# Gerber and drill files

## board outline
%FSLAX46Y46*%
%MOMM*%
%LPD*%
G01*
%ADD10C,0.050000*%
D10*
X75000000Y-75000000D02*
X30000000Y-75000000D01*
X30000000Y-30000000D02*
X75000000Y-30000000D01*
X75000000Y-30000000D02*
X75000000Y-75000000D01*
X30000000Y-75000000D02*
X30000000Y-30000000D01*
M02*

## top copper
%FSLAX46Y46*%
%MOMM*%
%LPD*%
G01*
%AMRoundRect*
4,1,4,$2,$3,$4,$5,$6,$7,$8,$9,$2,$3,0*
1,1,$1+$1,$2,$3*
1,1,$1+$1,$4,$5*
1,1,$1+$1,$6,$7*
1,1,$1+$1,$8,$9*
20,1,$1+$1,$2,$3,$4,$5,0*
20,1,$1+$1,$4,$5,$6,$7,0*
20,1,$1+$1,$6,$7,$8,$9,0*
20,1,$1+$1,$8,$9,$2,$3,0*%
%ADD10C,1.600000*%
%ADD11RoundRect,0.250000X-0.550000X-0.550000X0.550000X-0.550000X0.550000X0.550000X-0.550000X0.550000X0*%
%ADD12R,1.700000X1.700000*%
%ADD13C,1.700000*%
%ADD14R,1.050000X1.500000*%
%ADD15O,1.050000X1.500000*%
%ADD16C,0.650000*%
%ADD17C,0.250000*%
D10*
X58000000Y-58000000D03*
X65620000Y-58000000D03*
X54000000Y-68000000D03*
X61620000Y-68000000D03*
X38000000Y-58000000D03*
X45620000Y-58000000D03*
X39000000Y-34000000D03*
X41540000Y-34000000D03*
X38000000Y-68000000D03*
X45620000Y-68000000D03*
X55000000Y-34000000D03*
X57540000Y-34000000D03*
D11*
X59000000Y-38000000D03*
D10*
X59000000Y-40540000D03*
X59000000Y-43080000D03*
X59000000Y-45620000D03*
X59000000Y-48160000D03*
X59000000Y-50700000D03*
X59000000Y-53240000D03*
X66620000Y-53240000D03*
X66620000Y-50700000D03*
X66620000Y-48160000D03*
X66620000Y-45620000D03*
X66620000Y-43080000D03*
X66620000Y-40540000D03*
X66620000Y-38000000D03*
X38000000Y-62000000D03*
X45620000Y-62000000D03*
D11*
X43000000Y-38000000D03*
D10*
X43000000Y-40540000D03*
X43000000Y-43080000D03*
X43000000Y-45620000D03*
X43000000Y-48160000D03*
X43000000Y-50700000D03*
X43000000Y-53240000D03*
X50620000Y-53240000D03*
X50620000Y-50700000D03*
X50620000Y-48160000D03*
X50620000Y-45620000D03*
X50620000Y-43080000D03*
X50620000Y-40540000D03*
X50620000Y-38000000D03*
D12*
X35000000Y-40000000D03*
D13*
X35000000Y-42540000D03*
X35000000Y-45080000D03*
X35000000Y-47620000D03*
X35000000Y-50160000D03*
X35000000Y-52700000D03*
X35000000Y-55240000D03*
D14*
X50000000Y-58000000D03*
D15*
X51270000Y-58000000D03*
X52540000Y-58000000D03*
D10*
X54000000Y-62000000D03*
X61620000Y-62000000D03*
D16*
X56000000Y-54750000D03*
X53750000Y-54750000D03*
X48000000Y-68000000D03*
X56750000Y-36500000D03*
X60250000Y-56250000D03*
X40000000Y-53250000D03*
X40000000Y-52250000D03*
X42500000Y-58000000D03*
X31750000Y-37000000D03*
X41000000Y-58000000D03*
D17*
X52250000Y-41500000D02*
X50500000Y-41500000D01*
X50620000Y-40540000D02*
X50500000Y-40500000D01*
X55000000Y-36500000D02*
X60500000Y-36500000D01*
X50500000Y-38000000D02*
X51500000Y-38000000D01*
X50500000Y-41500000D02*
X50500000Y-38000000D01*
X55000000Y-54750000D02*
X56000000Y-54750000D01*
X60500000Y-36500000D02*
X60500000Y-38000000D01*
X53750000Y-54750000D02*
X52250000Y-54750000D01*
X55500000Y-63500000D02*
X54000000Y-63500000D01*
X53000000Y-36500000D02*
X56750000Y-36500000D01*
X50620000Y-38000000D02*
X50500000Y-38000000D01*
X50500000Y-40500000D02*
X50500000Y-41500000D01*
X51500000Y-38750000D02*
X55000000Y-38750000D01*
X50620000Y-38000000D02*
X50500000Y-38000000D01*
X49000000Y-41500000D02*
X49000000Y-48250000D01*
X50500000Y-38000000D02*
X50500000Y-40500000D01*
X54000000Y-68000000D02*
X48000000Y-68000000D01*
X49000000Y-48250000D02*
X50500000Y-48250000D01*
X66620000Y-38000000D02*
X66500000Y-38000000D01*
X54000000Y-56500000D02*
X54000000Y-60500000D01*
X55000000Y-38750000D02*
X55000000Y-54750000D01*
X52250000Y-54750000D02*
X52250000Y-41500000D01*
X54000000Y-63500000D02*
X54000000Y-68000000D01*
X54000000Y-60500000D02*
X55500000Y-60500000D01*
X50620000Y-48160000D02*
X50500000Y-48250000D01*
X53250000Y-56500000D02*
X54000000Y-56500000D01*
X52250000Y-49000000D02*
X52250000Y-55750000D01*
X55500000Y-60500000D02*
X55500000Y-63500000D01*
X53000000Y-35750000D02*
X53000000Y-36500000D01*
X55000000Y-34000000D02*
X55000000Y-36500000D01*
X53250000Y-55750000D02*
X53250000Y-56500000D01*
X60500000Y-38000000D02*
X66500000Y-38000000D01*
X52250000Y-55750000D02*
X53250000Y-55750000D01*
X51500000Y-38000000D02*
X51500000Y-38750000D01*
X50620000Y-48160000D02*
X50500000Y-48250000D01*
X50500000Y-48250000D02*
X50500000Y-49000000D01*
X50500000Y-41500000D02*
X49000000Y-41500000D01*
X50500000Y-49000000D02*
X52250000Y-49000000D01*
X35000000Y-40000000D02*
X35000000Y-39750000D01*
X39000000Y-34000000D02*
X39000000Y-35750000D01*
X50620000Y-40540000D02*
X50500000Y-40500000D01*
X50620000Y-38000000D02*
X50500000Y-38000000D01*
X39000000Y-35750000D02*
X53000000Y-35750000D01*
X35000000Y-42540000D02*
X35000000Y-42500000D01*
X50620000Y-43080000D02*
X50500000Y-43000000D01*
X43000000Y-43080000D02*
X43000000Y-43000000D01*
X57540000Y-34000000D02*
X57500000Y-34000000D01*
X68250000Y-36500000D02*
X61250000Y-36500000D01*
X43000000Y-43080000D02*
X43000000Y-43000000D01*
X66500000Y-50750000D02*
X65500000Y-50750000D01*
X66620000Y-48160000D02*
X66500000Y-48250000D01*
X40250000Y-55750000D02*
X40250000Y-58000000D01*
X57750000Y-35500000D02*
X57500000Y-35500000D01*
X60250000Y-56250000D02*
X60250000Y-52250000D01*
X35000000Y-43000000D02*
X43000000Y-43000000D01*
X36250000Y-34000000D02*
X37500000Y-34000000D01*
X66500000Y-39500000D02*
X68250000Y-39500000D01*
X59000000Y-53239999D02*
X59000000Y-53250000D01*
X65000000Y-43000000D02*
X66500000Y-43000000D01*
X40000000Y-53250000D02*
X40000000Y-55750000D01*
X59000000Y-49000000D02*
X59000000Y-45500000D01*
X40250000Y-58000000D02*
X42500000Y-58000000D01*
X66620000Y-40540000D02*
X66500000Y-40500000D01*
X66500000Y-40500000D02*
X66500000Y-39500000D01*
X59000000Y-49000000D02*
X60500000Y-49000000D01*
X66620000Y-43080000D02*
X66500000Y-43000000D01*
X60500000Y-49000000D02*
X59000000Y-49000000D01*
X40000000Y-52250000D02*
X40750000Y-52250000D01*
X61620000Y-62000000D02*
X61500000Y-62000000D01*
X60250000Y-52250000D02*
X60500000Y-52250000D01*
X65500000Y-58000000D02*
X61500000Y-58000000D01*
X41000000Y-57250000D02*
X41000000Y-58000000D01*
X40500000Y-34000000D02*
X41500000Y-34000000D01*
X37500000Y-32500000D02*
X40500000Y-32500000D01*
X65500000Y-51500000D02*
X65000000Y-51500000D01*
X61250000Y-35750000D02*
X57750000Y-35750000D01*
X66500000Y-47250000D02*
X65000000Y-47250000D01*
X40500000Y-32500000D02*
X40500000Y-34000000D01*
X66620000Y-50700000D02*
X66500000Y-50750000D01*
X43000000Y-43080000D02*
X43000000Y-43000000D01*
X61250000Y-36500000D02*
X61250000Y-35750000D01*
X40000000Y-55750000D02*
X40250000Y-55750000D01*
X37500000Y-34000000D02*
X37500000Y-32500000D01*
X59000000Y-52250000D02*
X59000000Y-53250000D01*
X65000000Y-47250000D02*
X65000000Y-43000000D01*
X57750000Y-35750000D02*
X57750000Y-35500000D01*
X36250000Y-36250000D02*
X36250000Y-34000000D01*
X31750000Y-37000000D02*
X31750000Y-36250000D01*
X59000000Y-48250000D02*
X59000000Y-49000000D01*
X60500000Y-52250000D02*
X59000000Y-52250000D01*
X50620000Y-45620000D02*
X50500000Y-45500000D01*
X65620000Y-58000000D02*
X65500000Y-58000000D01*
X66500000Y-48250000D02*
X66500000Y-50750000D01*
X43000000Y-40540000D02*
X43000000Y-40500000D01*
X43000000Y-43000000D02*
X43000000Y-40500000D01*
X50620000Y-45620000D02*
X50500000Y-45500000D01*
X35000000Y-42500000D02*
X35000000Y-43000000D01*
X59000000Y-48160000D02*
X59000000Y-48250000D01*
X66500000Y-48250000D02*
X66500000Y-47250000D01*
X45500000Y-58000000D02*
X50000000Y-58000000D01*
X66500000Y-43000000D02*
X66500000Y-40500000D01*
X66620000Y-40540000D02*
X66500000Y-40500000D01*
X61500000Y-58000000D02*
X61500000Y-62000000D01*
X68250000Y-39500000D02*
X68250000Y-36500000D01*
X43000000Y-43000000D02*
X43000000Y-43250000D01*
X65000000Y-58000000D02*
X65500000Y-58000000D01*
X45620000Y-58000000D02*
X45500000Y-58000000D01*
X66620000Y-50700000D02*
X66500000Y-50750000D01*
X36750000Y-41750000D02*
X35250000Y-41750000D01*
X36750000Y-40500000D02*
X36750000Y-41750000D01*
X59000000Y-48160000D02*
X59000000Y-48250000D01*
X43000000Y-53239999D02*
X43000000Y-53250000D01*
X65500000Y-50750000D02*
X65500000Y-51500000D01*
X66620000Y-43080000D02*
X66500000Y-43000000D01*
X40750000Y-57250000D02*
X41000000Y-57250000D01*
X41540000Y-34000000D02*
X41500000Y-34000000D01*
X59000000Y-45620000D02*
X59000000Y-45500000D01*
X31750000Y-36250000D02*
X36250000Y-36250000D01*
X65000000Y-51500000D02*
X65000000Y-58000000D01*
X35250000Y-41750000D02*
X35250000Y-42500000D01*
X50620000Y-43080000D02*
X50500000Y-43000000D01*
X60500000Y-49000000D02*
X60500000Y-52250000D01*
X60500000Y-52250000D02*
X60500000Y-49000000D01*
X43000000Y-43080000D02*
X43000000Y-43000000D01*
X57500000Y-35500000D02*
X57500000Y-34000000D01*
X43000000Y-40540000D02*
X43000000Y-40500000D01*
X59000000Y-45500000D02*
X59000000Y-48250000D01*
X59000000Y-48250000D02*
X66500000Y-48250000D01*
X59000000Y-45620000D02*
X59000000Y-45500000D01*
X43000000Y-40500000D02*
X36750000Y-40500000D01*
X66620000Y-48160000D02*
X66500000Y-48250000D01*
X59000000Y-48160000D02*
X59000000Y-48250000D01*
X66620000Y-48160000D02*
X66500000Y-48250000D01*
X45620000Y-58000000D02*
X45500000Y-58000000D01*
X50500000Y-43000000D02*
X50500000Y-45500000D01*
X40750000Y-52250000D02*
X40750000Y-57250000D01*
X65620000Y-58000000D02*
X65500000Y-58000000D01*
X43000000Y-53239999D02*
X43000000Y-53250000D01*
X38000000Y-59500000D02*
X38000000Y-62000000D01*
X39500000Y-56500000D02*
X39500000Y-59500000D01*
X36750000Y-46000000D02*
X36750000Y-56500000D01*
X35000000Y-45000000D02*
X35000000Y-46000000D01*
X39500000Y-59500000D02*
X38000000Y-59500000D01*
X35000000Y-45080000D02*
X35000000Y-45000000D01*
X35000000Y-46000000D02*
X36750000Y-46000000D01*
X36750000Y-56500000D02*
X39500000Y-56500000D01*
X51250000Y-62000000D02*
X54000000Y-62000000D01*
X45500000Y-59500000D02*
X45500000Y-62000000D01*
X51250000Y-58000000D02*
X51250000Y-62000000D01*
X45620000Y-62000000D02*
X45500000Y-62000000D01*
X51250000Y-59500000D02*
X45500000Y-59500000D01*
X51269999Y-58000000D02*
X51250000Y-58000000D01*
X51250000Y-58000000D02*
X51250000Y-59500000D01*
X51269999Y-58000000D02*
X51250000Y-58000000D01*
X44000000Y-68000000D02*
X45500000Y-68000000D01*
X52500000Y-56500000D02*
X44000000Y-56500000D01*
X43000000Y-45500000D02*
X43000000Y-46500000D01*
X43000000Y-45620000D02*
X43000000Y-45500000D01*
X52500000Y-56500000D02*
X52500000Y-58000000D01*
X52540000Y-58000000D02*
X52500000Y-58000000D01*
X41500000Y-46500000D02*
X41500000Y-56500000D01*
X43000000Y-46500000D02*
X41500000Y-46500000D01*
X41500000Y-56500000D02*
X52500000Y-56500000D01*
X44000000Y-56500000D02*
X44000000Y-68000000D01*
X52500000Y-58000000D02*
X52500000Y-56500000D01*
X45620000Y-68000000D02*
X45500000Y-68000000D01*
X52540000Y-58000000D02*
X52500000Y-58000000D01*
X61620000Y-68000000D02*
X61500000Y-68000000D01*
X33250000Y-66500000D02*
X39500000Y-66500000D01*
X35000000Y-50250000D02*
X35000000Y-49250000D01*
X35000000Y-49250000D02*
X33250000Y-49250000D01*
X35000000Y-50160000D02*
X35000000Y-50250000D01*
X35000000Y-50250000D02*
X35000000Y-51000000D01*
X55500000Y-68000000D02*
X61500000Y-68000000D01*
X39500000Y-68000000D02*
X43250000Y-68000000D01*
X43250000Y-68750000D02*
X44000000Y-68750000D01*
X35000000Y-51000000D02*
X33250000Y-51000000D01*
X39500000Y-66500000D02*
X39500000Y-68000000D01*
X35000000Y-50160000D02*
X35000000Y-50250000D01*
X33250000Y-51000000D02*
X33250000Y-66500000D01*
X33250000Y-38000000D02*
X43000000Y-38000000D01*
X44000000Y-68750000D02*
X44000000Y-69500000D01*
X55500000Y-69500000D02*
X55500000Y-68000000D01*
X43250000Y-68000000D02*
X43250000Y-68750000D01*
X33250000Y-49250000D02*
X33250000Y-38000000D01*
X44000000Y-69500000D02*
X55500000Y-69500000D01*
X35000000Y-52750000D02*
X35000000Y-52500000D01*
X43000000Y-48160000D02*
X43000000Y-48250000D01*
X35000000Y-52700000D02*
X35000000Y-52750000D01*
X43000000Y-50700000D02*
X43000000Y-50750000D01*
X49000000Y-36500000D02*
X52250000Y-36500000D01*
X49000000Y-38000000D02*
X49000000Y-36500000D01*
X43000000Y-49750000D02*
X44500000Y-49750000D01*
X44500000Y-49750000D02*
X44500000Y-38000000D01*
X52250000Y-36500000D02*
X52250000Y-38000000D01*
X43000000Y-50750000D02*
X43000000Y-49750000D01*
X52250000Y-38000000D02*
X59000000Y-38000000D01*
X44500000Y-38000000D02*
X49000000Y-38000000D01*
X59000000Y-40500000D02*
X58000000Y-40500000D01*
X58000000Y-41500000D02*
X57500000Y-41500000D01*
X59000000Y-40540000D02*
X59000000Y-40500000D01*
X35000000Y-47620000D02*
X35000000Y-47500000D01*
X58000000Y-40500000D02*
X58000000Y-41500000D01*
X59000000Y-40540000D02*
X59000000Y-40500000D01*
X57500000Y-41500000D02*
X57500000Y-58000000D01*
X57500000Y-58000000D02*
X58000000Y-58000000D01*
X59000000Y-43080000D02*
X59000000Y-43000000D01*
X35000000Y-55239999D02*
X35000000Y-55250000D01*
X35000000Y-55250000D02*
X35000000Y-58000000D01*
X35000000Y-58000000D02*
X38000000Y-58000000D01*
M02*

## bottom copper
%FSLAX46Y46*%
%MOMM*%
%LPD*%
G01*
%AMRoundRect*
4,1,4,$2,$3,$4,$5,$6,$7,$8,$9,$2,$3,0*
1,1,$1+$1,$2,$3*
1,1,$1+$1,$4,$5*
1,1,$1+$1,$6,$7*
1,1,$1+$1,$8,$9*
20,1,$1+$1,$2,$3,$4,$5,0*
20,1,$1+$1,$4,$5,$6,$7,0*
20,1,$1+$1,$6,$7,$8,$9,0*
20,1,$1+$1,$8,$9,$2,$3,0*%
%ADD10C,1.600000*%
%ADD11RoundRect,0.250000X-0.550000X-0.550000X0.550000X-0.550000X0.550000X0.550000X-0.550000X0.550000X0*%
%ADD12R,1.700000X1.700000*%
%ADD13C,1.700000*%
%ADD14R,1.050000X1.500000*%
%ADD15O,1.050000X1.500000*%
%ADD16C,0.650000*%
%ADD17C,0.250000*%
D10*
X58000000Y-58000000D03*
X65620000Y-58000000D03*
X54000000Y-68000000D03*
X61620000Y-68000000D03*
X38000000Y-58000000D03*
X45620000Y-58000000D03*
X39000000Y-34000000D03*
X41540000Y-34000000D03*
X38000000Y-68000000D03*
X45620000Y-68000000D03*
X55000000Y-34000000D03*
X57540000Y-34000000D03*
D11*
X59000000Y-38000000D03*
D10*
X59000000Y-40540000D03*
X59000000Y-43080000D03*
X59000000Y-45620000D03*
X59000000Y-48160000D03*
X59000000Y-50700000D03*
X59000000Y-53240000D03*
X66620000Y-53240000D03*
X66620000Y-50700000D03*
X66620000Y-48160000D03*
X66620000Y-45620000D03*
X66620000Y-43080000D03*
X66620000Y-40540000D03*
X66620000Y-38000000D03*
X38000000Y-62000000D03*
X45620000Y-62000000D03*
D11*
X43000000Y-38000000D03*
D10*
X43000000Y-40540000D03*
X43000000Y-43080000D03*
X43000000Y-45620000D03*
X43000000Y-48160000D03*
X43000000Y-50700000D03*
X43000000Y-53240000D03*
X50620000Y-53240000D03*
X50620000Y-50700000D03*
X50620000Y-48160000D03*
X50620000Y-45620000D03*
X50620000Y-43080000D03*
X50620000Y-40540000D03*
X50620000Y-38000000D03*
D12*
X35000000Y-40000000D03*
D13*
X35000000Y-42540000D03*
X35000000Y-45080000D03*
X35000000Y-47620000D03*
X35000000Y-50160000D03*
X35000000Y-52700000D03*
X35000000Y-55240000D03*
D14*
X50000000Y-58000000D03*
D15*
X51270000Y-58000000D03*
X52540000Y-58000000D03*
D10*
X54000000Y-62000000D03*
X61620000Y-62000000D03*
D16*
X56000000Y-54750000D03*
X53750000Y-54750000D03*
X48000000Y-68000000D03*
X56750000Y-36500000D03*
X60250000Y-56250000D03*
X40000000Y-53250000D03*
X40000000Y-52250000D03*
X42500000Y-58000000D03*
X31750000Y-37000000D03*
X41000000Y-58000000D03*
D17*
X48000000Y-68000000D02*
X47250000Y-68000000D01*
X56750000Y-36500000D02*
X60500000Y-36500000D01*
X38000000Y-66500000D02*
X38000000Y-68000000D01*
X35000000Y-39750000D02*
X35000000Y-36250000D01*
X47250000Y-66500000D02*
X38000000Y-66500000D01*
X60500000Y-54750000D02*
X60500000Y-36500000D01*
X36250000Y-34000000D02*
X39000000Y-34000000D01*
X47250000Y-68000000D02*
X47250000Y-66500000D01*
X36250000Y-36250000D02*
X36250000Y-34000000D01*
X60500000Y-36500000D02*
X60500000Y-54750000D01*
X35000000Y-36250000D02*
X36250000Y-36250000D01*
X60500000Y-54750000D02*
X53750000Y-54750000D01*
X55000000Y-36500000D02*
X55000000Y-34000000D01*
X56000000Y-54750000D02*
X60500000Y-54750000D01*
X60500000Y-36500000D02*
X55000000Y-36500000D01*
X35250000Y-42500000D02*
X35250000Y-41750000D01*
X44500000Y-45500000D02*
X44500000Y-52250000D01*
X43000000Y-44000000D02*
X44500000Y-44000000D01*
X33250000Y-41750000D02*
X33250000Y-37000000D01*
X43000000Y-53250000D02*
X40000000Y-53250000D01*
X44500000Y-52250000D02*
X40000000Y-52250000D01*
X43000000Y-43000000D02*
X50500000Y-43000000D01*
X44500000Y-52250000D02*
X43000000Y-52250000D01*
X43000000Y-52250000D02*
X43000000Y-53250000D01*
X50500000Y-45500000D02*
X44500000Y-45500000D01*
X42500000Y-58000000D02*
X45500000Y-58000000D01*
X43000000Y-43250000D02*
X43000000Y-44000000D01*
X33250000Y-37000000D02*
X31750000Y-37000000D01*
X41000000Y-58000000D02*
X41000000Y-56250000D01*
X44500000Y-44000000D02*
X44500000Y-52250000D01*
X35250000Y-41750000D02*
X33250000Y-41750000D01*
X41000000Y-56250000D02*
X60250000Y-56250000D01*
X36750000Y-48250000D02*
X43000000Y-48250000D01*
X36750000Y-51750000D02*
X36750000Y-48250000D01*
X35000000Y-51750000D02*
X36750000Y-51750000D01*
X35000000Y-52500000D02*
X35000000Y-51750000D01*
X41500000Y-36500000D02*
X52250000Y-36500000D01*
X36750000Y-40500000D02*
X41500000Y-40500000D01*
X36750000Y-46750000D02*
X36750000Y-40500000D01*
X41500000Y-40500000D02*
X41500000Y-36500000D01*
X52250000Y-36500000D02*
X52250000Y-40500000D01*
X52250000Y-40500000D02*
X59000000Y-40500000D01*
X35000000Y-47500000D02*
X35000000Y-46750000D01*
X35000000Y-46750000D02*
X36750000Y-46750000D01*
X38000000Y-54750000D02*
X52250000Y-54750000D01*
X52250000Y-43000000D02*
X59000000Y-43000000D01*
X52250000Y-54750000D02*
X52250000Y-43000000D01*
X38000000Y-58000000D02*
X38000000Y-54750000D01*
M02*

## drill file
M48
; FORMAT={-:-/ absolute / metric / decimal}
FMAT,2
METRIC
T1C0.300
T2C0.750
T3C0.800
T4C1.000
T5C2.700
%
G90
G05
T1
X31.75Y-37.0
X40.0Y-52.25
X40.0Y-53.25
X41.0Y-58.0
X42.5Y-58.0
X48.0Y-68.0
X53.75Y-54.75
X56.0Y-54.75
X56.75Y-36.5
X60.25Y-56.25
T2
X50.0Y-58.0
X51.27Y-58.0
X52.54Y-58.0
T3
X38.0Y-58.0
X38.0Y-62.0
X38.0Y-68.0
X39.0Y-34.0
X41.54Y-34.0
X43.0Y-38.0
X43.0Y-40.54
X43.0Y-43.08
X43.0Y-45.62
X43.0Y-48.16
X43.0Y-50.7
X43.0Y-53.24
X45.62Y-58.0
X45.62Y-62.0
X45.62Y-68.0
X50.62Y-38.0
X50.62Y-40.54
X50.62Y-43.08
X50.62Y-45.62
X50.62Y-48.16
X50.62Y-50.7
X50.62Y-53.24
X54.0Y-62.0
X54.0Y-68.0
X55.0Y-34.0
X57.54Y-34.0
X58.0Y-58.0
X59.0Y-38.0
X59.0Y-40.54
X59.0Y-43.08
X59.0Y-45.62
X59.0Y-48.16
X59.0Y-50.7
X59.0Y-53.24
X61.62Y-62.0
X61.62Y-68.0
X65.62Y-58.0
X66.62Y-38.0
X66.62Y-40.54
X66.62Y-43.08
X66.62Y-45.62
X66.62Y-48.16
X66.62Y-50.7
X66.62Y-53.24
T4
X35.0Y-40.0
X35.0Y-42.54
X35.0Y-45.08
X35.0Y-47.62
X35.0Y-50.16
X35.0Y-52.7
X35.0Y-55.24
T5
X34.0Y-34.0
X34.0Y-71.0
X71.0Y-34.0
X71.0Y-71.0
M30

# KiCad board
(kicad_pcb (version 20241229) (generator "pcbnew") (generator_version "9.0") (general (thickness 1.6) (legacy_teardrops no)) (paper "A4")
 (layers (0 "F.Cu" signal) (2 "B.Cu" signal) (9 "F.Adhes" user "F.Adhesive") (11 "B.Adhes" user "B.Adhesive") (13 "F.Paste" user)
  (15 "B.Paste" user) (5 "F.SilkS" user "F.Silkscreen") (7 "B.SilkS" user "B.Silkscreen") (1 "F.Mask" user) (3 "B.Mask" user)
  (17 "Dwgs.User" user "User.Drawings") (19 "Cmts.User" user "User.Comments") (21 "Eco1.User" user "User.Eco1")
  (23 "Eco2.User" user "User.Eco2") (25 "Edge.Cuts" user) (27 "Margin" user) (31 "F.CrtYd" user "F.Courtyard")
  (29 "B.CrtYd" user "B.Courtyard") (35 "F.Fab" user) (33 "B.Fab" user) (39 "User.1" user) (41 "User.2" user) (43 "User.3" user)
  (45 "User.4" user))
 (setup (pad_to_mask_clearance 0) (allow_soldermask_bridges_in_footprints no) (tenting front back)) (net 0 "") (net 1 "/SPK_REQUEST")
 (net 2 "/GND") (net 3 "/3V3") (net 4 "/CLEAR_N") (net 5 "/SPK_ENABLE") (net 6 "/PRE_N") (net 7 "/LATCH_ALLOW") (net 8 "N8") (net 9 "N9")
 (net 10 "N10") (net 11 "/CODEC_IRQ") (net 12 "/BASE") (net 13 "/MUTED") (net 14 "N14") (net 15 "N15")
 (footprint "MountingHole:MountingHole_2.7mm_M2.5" (layer "F.Cu") (at 34 71)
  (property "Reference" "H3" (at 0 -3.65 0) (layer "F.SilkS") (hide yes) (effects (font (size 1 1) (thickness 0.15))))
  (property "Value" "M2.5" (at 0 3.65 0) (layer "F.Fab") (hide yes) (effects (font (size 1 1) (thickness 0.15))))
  (pad "" np_thru_hole circle (at 0 0) (size 2.7 2.7) (drill 2.7) (layers "*.Cu" "*.Mask")))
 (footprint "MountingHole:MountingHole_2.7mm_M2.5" (layer "F.Cu") (at 71 71)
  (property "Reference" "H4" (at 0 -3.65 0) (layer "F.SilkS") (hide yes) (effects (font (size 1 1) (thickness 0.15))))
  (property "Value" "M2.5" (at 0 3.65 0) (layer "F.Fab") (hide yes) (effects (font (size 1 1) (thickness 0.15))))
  (pad "" np_thru_hole circle (at 0 0) (size 2.7 2.7) (drill 2.7) (layers "*.Cu" "*.Mask")))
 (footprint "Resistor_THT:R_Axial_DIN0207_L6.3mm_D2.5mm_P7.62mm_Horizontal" (layer "F.Cu") (at 58 58)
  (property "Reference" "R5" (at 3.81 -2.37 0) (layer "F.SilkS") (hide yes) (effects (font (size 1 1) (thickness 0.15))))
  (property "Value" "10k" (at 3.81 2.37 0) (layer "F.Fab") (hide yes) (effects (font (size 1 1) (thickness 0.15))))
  (pad "1" thru_hole circle (at 0 0) (size 1.6 1.6) (drill 0.8) (layers "*.Cu" "*.Mask") (remove_unused_layers no) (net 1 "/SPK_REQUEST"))
  (pad "2" thru_hole circle (at 7.62 0) (size 1.6 1.6) (drill 0.8) (layers "*.Cu" "*.Mask") (remove_unused_layers no) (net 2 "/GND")))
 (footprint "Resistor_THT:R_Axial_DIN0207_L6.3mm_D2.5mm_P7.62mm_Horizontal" (layer "F.Cu") (at 54 68)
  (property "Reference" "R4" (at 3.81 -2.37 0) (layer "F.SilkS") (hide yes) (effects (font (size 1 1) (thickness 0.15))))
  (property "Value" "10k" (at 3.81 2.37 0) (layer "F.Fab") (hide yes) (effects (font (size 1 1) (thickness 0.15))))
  (pad "1" thru_hole circle (at 0 0) (size 1.6 1.6) (drill 0.8) (layers "*.Cu" "*.Mask") (remove_unused_layers no) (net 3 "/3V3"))
  (pad "2" thru_hole circle (at 7.62 0) (size 1.6 1.6) (drill 0.8) (layers "*.Cu" "*.Mask") (remove_unused_layers no) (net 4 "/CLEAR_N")))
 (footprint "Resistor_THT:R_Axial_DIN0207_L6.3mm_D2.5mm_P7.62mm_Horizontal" (layer "F.Cu") (at 38 58)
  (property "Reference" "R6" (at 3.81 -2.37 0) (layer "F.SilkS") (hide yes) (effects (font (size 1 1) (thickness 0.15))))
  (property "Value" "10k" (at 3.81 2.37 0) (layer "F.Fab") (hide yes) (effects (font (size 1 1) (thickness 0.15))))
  (pad "1" thru_hole circle (at 0 0) (size 1.6 1.6) (drill 0.8) (layers "*.Cu" "*.Mask") (remove_unused_layers no) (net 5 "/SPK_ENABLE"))
  (pad "2" thru_hole circle (at 7.62 0) (size 1.6 1.6) (drill 0.8) (layers "*.Cu" "*.Mask") (remove_unused_layers no) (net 2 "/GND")))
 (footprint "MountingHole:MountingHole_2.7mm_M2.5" (layer "F.Cu") (at 34 34)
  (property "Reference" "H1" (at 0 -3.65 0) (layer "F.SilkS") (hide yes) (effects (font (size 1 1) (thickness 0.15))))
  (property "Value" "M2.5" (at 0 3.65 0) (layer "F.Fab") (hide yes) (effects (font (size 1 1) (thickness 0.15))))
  (pad "" np_thru_hole circle (at 0 0) (size 2.7 2.7) (drill 2.7) (layers "*.Cu" "*.Mask")))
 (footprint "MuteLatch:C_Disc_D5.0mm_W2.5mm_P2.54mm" (layer "F.Cu") (at 39 34)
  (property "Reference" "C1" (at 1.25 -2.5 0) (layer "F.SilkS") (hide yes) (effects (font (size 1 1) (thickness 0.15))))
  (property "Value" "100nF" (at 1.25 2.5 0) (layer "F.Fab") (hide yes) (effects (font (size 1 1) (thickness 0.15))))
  (pad "1" thru_hole circle (at 0 0) (size 1.6 1.6) (drill 0.8) (layers "*.Cu" "*.Mask") (remove_unused_layers no) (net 3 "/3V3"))
  (pad "2" thru_hole circle (at 2.54 0) (size 1.6 1.6) (drill 0.8) (layers "*.Cu" "*.Mask") (remove_unused_layers no) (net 2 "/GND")))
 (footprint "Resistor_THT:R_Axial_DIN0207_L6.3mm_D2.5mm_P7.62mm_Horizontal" (layer "F.Cu") (at 38 68)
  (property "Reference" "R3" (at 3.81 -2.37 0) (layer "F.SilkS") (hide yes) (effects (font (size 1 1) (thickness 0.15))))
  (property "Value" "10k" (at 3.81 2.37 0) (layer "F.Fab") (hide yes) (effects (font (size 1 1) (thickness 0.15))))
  (pad "1" thru_hole circle (at 0 0) (size 1.6 1.6) (drill 0.8) (layers "*.Cu" "*.Mask") (remove_unused_layers no) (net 3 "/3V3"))
  (pad "2" thru_hole circle (at 7.62 0) (size 1.6 1.6) (drill 0.8) (layers "*.Cu" "*.Mask") (remove_unused_layers no) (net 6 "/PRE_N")))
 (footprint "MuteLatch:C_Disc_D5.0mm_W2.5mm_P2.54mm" (layer "F.Cu") (at 55 34)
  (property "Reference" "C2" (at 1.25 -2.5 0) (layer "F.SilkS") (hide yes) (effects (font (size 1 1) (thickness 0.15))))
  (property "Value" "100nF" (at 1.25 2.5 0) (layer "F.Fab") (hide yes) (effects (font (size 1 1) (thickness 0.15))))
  (pad "1" thru_hole circle (at 0 0) (size 1.6 1.6) (drill 0.8) (layers "*.Cu" "*.Mask") (remove_unused_layers no) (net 3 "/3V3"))
  (pad "2" thru_hole circle (at 2.54 0) (size 1.6 1.6) (drill 0.8) (layers "*.Cu" "*.Mask") (remove_unused_layers no) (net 2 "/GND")))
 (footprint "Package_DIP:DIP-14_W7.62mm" (layer "F.Cu") (at 59 38)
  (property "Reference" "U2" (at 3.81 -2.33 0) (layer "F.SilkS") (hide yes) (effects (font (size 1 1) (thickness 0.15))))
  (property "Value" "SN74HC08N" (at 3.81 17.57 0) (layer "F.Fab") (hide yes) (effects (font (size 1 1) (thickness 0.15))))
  (pad "1" thru_hole roundrect (at 0 0) (size 1.6 1.6) (drill 0.8) (layers "*.Cu" "*.Mask") (remove_unused_layers no)
   (roundrect_rratio 0.15625) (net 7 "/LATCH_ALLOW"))
  (pad "2" thru_hole circle (at 0 2.54) (size 1.6 1.6) (drill 0.8) (layers "*.Cu" "*.Mask") (remove_unused_layers no) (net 1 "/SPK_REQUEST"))
  (pad "3" thru_hole circle (at 0 5.08) (size 1.6 1.6) (drill 0.8) (layers "*.Cu" "*.Mask") (remove_unused_layers no) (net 5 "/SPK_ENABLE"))
  (pad "4" thru_hole circle (at 0 7.62) (size 1.6 1.6) (drill 0.8) (layers "*.Cu" "*.Mask") (remove_unused_layers no) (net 2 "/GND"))
  (pad "5" thru_hole circle (at 0 10.16) (size 1.6 1.6) (drill 0.8) (layers "*.Cu" "*.Mask") (remove_unused_layers no) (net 2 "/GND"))
  (pad "6" thru_hole circle (at 0 12.7) (size 1.6 1.6) (drill 0.8) (layers "*.Cu" "*.Mask") (remove_unused_layers no) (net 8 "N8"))
  (pad "7" thru_hole circle (at 0 15.24) (size 1.6 1.6) (drill 0.8) (layers "*.Cu" "*.Mask") (remove_unused_layers no) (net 2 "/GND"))
  (pad "8" thru_hole circle (at 7.62 15.24) (size 1.6 1.6) (drill 0.8) (layers "*.Cu" "*.Mask") (remove_unused_layers no) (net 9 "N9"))
  (pad "9" thru_hole circle (at 7.62 12.7) (size 1.6 1.6) (drill 0.8) (layers "*.Cu" "*.Mask") (remove_unused_layers no) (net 2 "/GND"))
  (pad "10" thru_hole circle (at 7.62 10.16) (size 1.6 1.6) (drill 0.8) (layers "*.Cu" "*.Mask") (remove_unused_layers no) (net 2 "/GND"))
  (pad "11" thru_hole circle (at 7.62 7.62) (size 1.6 1.6) (drill 0.8) (layers "*.Cu" "*.Mask") (remove_unused_layers no) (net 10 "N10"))
  (pad "12" thru_hole circle (at 7.62 5.08) (size 1.6 1.6) (drill 0.8) (layers "*.Cu" "*.Mask") (remove_unused_layers no) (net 2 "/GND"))
  (pad "13" thru_hole circle (at 7.62 2.54) (size 1.6 1.6) (drill 0.8) (layers "*.Cu" "*.Mask") (remove_unused_layers no) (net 2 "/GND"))
  (pad "14" thru_hole circle (at 7.62 0) (size 1.6 1.6) (drill 0.8) (layers "*.Cu" "*.Mask") (remove_unused_layers no) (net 3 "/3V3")))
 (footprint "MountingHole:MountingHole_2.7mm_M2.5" (layer "F.Cu") (at 71 34)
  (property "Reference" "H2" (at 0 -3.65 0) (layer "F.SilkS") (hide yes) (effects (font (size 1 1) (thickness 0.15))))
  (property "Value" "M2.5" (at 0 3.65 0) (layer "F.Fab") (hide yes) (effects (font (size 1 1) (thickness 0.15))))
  (pad "" np_thru_hole circle (at 0 0) (size 2.7 2.7) (drill 2.7) (layers "*.Cu" "*.Mask")))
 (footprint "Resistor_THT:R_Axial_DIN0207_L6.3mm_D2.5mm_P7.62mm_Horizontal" (layer "F.Cu") (at 38 62)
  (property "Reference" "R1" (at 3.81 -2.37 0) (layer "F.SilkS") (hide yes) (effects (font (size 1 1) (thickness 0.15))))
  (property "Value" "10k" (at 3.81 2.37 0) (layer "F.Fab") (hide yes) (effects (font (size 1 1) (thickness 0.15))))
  (pad "1" thru_hole circle (at 0 0) (size 1.6 1.6) (drill 0.8) (layers "*.Cu" "*.Mask") (remove_unused_layers no) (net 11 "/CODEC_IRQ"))
  (pad "2" thru_hole circle (at 7.62 0) (size 1.6 1.6) (drill 0.8) (layers "*.Cu" "*.Mask") (remove_unused_layers no) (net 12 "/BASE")))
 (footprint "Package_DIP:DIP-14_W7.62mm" (layer "F.Cu") (at 43 38)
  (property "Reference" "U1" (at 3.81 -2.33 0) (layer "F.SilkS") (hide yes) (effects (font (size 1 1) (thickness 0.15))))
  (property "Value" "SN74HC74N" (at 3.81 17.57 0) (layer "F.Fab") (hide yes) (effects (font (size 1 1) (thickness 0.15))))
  (pad "1" thru_hole roundrect (at 0 0) (size 1.6 1.6) (drill 0.8) (layers "*.Cu" "*.Mask") (remove_unused_layers no)
   (roundrect_rratio 0.15625) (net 4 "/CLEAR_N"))
  (pad "2" thru_hole circle (at 0 2.54) (size 1.6 1.6) (drill 0.8) (layers "*.Cu" "*.Mask") (remove_unused_layers no) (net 2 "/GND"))
  (pad "3" thru_hole circle (at 0 5.08) (size 1.6 1.6) (drill 0.8) (layers "*.Cu" "*.Mask") (remove_unused_layers no) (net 2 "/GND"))
  (pad "4" thru_hole circle (at 0 7.62) (size 1.6 1.6) (drill 0.8) (layers "*.Cu" "*.Mask") (remove_unused_layers no) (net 6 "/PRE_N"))
  (pad "5" thru_hole circle (at 0 10.16) (size 1.6 1.6) (drill 0.8) (layers "*.Cu" "*.Mask") (remove_unused_layers no) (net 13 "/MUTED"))
  (pad "6" thru_hole circle (at 0 12.7) (size 1.6 1.6) (drill 0.8) (layers "*.Cu" "*.Mask") (remove_unused_layers no) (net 7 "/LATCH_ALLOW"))
  (pad "7" thru_hole circle (at 0 15.24) (size 1.6 1.6) (drill 0.8) (layers "*.Cu" "*.Mask") (remove_unused_layers no) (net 2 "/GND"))
  (pad "8" thru_hole circle (at 7.62 15.24) (size 1.6 1.6) (drill 0.8) (layers "*.Cu" "*.Mask") (remove_unused_layers no) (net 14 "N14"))
  (pad "9" thru_hole circle (at 7.62 12.7) (size 1.6 1.6) (drill 0.8) (layers "*.Cu" "*.Mask") (remove_unused_layers no) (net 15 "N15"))
  (pad "10" thru_hole circle (at 7.62 10.16) (size 1.6 1.6) (drill 0.8) (layers "*.Cu" "*.Mask") (remove_unused_layers no) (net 3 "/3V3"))
  (pad "11" thru_hole circle (at 7.62 7.62) (size 1.6 1.6) (drill 0.8) (layers "*.Cu" "*.Mask") (remove_unused_layers no) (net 2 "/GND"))
  (pad "12" thru_hole circle (at 7.62 5.08) (size 1.6 1.6) (drill 0.8) (layers "*.Cu" "*.Mask") (remove_unused_layers no) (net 2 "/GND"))
  (pad "13" thru_hole circle (at 7.62 2.54) (size 1.6 1.6) (drill 0.8) (layers "*.Cu" "*.Mask") (remove_unused_layers no) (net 3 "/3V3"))
  (pad "14" thru_hole circle (at 7.62 0) (size 1.6 1.6) (drill 0.8) (layers "*.Cu" "*.Mask") (remove_unused_layers no) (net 3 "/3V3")))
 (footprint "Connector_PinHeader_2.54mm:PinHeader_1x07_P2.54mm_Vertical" (layer "F.Cu") (at 35 40)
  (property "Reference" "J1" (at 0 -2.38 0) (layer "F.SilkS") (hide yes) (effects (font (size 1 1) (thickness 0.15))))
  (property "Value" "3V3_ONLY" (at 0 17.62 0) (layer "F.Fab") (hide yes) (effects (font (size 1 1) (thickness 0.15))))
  (pad "1" thru_hole rect (at 0 0) (size 1.7 1.7) (drill 1) (layers "*.Cu" "*.Mask") (remove_unused_layers no) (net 3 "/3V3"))
  (pad "2" thru_hole circle (at 0 2.54) (size 1.7 1.7) (drill 1) (layers "*.Cu" "*.Mask") (remove_unused_layers no) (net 2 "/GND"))
  (pad "3" thru_hole circle (at 0 5.08) (size 1.7 1.7) (drill 1) (layers "*.Cu" "*.Mask") (remove_unused_layers no) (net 11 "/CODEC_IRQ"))
  (pad "4" thru_hole circle (at 0 7.62) (size 1.7 1.7) (drill 1) (layers "*.Cu" "*.Mask") (remove_unused_layers no) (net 1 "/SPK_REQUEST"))
  (pad "5" thru_hole circle (at 0 10.16) (size 1.7 1.7) (drill 1) (layers "*.Cu" "*.Mask") (remove_unused_layers no) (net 4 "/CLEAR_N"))
  (pad "6" thru_hole circle (at 0 12.7) (size 1.7 1.7) (drill 1) (layers "*.Cu" "*.Mask") (remove_unused_layers no) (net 13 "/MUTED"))
  (pad "7" thru_hole circle (at 0 15.24) (size 1.7 1.7) (drill 1) (layers "*.Cu" "*.Mask") (remove_unused_layers no) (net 5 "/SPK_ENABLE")))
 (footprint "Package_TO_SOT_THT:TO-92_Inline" (layer "F.Cu") (at 50 58)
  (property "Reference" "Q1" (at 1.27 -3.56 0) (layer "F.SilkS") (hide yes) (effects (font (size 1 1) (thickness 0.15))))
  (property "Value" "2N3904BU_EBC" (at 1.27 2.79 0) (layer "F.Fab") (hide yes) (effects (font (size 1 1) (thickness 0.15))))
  (pad "1" thru_hole rect (at 0 0) (size 1.05 1.5) (drill 0.75) (layers "*.Cu" "*.Mask") (remove_unused_layers no) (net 2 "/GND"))
  (pad "2" thru_hole oval (at 1.27 0) (size 1.05 1.5) (drill 0.75) (layers "*.Cu" "*.Mask") (remove_unused_layers no) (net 12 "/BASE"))
  (pad "3" thru_hole oval (at 2.54 0) (size 1.05 1.5) (drill 0.75) (layers "*.Cu" "*.Mask") (remove_unused_layers no) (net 6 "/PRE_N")))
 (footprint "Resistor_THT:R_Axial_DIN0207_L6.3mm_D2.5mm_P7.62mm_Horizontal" (layer "F.Cu") (at 54 62)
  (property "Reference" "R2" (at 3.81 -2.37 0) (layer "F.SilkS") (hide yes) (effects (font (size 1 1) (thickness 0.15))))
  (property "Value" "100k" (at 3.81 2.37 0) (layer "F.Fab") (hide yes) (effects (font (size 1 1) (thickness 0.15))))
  (pad "1" thru_hole circle (at 0 0) (size 1.6 1.6) (drill 0.8) (layers "*.Cu" "*.Mask") (remove_unused_layers no) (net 12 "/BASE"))
  (pad "2" thru_hole circle (at 7.62 0) (size 1.6 1.6) (drill 0.8) (layers "*.Cu" "*.Mask") (remove_unused_layers no) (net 2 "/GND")))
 (gr_line (start 75 75) (end 30 75) (stroke (width 0.05) (type default)) (layer "Edge.Cuts"))
 (gr_line (start 30 30) (end 75 30) (stroke (width 0.05) (type default)) (layer "Edge.Cuts"))
 (gr_line (start 75 30) (end 75 75) (stroke (width 0.05) (type default)) (layer "Edge.Cuts"))
 (gr_line (start 30 75) (end 30 30) (stroke (width 0.05) (type default)) (layer "Edge.Cuts"))
 (segment (start 52.25 41.5) (end 50.5 41.5) (width 0.25) (layer "F.Cu") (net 3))
 (segment (start 50.62 40.54) (end 50.5 40.5) (width 0.25) (layer "F.Cu") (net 3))
 (segment (start 55 36.5) (end 60.5 36.5) (width 0.25) (layer "F.Cu") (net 3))
 (segment (start 50.5 38) (end 51.5 38) (width 0.25) (layer "F.Cu") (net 3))
 (segment (start 50.5 41.5) (end 50.5 38) (width 0.25) (layer "F.Cu") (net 3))
 (segment (start 55 54.75) (end 56 54.75) (width 0.25) (layer "F.Cu") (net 3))
 (segment (start 60.5 36.5) (end 60.5 38) (width 0.25) (layer "F.Cu") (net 3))
 (segment (start 53.75 54.75) (end 52.25 54.75) (width 0.25) (layer "F.Cu") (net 3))
 (segment (start 55.5 63.5) (end 54 63.5) (width 0.25) (layer "F.Cu") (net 3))
 (segment (start 53 36.5) (end 56.75 36.5) (width 0.25) (layer "F.Cu") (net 3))
 (segment (start 50.62 38) (end 50.5 38) (width 0.25) (layer "F.Cu") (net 3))
 (segment (start 50.5 40.5) (end 50.5 41.5) (width 0.25) (layer "F.Cu") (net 3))
 (segment (start 51.5 38.75) (end 55 38.75) (width 0.25) (layer "F.Cu") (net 3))
 (segment (start 50.62 38) (end 50.5 38) (width 0.25) (layer "F.Cu") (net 3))
 (segment (start 49 41.5) (end 49 48.25) (width 0.25) (layer "F.Cu") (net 3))
 (segment (start 50.5 38) (end 50.5 40.5) (width 0.25) (layer "F.Cu") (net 3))
 (segment (start 54 68) (end 48 68) (width 0.25) (layer "F.Cu") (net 3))
 (segment (start 49 48.25) (end 50.5 48.25) (width 0.25) (layer "F.Cu") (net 3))
 (segment (start 66.62 38) (end 66.5 38) (width 0.25) (layer "F.Cu") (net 3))
 (segment (start 54 56.5) (end 54 60.5) (width 0.25) (layer "F.Cu") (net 3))
 (segment (start 55 38.75) (end 55 54.75) (width 0.25) (layer "F.Cu") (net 3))
 (segment (start 52.25 54.75) (end 52.25 41.5) (width 0.25) (layer "F.Cu") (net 3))
 (segment (start 54 63.5) (end 54 68) (width 0.25) (layer "F.Cu") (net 3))
 (segment (start 54 60.5) (end 55.5 60.5) (width 0.25) (layer "F.Cu") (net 3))
 (segment (start 50.62 48.16) (end 50.5 48.25) (width 0.25) (layer "F.Cu") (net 3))
 (segment (start 53.25 56.5) (end 54 56.5) (width 0.25) (layer "F.Cu") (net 3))
 (segment (start 52.25 49) (end 52.25 55.75) (width 0.25) (layer "F.Cu") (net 3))
 (segment (start 55.5 60.5) (end 55.5 63.5) (width 0.25) (layer "F.Cu") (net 3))
 (segment (start 53 35.75) (end 53 36.5) (width 0.25) (layer "F.Cu") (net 3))
 (segment (start 55 34) (end 55 36.5) (width 0.25) (layer "F.Cu") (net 3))
 (segment (start 53.25 55.75) (end 53.25 56.5) (width 0.25) (layer "F.Cu") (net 3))
 (segment (start 60.5 38) (end 66.5 38) (width 0.25) (layer "F.Cu") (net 3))
 (segment (start 52.25 55.75) (end 53.25 55.75) (width 0.25) (layer "F.Cu") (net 3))
 (segment (start 51.5 38) (end 51.5 38.75) (width 0.25) (layer "F.Cu") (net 3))
 (segment (start 50.62 48.16) (end 50.5 48.25) (width 0.25) (layer "F.Cu") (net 3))
 (segment (start 50.5 48.25) (end 50.5 49) (width 0.25) (layer "F.Cu") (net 3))
 (segment (start 50.5 41.5) (end 49 41.5) (width 0.25) (layer "F.Cu") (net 3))
 (segment (start 50.5 49) (end 52.25 49) (width 0.25) (layer "F.Cu") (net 3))
 (segment (start 35 40) (end 35 39.75) (width 0.25) (layer "F.Cu") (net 3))
 (segment (start 39 34) (end 39 35.75) (width 0.25) (layer "F.Cu") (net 3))
 (segment (start 50.62 40.54) (end 50.5 40.5) (width 0.25) (layer "F.Cu") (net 3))
 (segment (start 50.62 38) (end 50.5 38) (width 0.25) (layer "F.Cu") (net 3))
 (segment (start 39 35.75) (end 53 35.75) (width 0.25) (layer "F.Cu") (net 3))
 (via (at 56 54.75) (size 0.65) (drill 0.3) (layers "F.Cu" "B.Cu") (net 3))
 (via (at 53.75 54.75) (size 0.65) (drill 0.3) (layers "F.Cu" "B.Cu") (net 3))
 (via (at 48 68) (size 0.65) (drill 0.3) (layers "F.Cu" "B.Cu") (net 3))
 (via (at 56.75 36.5) (size 0.65) (drill 0.3) (layers "F.Cu" "B.Cu") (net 3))
 (segment (start 48 68) (end 47.25 68) (width 0.25) (layer "B.Cu") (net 3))
 (segment (start 56.75 36.5) (end 60.5 36.5) (width 0.25) (layer "B.Cu") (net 3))
 (segment (start 38 66.5) (end 38 68) (width 0.25) (layer "B.Cu") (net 3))
 (segment (start 35 39.75) (end 35 36.25) (width 0.25) (layer "B.Cu") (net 3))
 (segment (start 47.25 66.5) (end 38 66.5) (width 0.25) (layer "B.Cu") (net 3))
 (segment (start 60.5 54.75) (end 60.5 36.5) (width 0.25) (layer "B.Cu") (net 3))
 (segment (start 36.25 34) (end 39 34) (width 0.25) (layer "B.Cu") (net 3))
 (segment (start 47.25 68) (end 47.25 66.5) (width 0.25) (layer "B.Cu") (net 3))
 (segment (start 36.25 36.25) (end 36.25 34) (width 0.25) (layer "B.Cu") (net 3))
 (segment (start 60.5 36.5) (end 60.5 54.75) (width 0.25) (layer "B.Cu") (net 3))
 (segment (start 35 36.25) (end 36.25 36.25) (width 0.25) (layer "B.Cu") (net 3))
 (segment (start 60.5 54.75) (end 53.75 54.75) (width 0.25) (layer "B.Cu") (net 3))
 (segment (start 55 36.5) (end 55 34) (width 0.25) (layer "B.Cu") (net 3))
 (segment (start 56 54.75) (end 60.5 54.75) (width 0.25) (layer "B.Cu") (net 3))
 (segment (start 60.5 36.5) (end 55 36.5) (width 0.25) (layer "B.Cu") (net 3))
 (segment (start 35 42.54) (end 35 42.5) (width 0.25) (layer "F.Cu") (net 2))
 (segment (start 50.62 43.08) (end 50.5 43) (width 0.25) (layer "F.Cu") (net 2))
 (segment (start 43 43.08) (end 43 43) (width 0.25) (layer "F.Cu") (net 2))
 (segment (start 57.54 34) (end 57.5 34) (width 0.25) (layer "F.Cu") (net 2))
 (segment (start 68.25 36.5) (end 61.25 36.5) (width 0.25) (layer "F.Cu") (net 2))
 (segment (start 43 43.08) (end 43 43) (width 0.25) (layer "F.Cu") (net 2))
 (segment (start 66.5 50.75) (end 65.5 50.75) (width 0.25) (layer "F.Cu") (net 2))
 (segment (start 66.62 48.16) (end 66.5 48.25) (width 0.25) (layer "F.Cu") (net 2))
 (segment (start 40.25 55.75) (end 40.25 58) (width 0.25) (layer "F.Cu") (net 2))
 (segment (start 57.75 35.5) (end 57.5 35.5) (width 0.25) (layer "F.Cu") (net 2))
 (segment (start 60.25 56.25) (end 60.25 52.25) (width 0.25) (layer "F.Cu") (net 2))
 (segment (start 35 43) (end 43 43) (width 0.25) (layer "F.Cu") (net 2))
 (segment (start 36.25 34) (end 37.5 34) (width 0.25) (layer "F.Cu") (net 2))
 (segment (start 66.5 39.5) (end 68.25 39.5) (width 0.25) (layer "F.Cu") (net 2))
 (segment (start 59 53.239999) (end 59 53.25) (width 0.25) (layer "F.Cu") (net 2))
 (segment (start 65 43) (end 66.5 43) (width 0.25) (layer "F.Cu") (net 2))
 (segment (start 40 53.25) (end 40 55.75) (width 0.25) (layer "F.Cu") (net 2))
 (segment (start 59 49) (end 59 45.5) (width 0.25) (layer "F.Cu") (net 2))
 (segment (start 40.25 58) (end 42.5 58) (width 0.25) (layer "F.Cu") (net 2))
 (segment (start 66.62 40.54) (end 66.5 40.5) (width 0.25) (layer "F.Cu") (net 2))
 (segment (start 66.5 40.5) (end 66.5 39.5) (width 0.25) (layer "F.Cu") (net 2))
 (segment (start 59 49) (end 60.5 49) (width 0.25) (layer "F.Cu") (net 2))
 (segment (start 66.62 43.08) (end 66.5 43) (width 0.25) (layer "F.Cu") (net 2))
 (segment (start 60.5 49) (end 59 49) (width 0.25) (layer "F.Cu") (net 2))
 (segment (start 40 52.25) (end 40.75 52.25) (width 0.25) (layer "F.Cu") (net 2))
 (segment (start 61.62 62) (end 61.5 62) (width 0.25) (layer "F.Cu") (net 2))
 (segment (start 60.25 52.25) (end 60.5 52.25) (width 0.25) (layer "F.Cu") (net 2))
 (segment (start 65.5 58) (end 61.5 58) (width 0.25) (layer "F.Cu") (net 2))
 (segment (start 41 57.25) (end 41 58) (width 0.25) (layer "F.Cu") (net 2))
 (segment (start 40.5 34) (end 41.5 34) (width 0.25) (layer "F.Cu") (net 2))
 (segment (start 37.5 32.5) (end 40.5 32.5) (width 0.25) (layer "F.Cu") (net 2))
 (segment (start 65.5 51.5) (end 65 51.5) (width 0.25) (layer "F.Cu") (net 2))
 (segment (start 61.25 35.75) (end 57.75 35.75) (width 0.25) (layer "F.Cu") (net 2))
 (segment (start 66.5 47.25) (end 65 47.25) (width 0.25) (layer "F.Cu") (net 2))
 (segment (start 40.5 32.5) (end 40.5 34) (width 0.25) (layer "F.Cu") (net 2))
 (segment (start 66.62 50.7) (end 66.5 50.75) (width 0.25) (layer "F.Cu") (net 2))
 (segment (start 43 43.08) (end 43 43) (width 0.25) (layer "F.Cu") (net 2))
 (segment (start 61.25 36.5) (end 61.25 35.75) (width 0.25) (layer "F.Cu") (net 2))
 (segment (start 40 55.75) (end 40.25 55.75) (width 0.25) (layer "F.Cu") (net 2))
 (segment (start 37.5 34) (end 37.5 32.5) (width 0.25) (layer "F.Cu") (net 2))
 (segment (start 59 52.25) (end 59 53.25) (width 0.25) (layer "F.Cu") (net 2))
 (segment (start 65 47.25) (end 65 43) (width 0.25) (layer "F.Cu") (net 2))
 (segment (start 57.75 35.75) (end 57.75 35.5) (width 0.25) (layer "F.Cu") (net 2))
 (segment (start 36.25 36.25) (end 36.25 34) (width 0.25) (layer "F.Cu") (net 2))
 (segment (start 31.75 37) (end 31.75 36.25) (width 0.25) (layer "F.Cu") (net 2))
 (segment (start 59 48.25) (end 59 49) (width 0.25) (layer "F.Cu") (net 2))
 (segment (start 60.5 52.25) (end 59 52.25) (width 0.25) (layer "F.Cu") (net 2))
 (segment (start 50.62 45.62) (end 50.5 45.5) (width 0.25) (layer "F.Cu") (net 2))
 (segment (start 65.62 58) (end 65.5 58) (width 0.25) (layer "F.Cu") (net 2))
 (segment (start 66.5 48.25) (end 66.5 50.75) (width 0.25) (layer "F.Cu") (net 2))
 (segment (start 43 40.54) (end 43 40.5) (width 0.25) (layer "F.Cu") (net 2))
 (segment (start 43 43) (end 43 40.5) (width 0.25) (layer "F.Cu") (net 2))
 (segment (start 50.62 45.62) (end 50.5 45.5) (width 0.25) (layer "F.Cu") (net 2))
 (segment (start 35 42.5) (end 35 43) (width 0.25) (layer "F.Cu") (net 2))
 (segment (start 59 48.16) (end 59 48.25) (width 0.25) (layer "F.Cu") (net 2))
 (segment (start 66.5 48.25) (end 66.5 47.25) (width 0.25) (layer "F.Cu") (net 2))
 (segment (start 45.5 58) (end 50 58) (width 0.25) (layer "F.Cu") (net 2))
 (segment (start 66.5 43) (end 66.5 40.5) (width 0.25) (layer "F.Cu") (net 2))
 (segment (start 66.62 40.54) (end 66.5 40.5) (width 0.25) (layer "F.Cu") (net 2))
 (segment (start 61.5 58) (end 61.5 62) (width 0.25) (layer "F.Cu") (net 2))
 (segment (start 68.25 39.5) (end 68.25 36.5) (width 0.25) (layer "F.Cu") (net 2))
 (segment (start 43 43) (end 43 43.25) (width 0.25) (layer "F.Cu") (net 2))
 (segment (start 65 58) (end 65.5 58) (width 0.25) (layer "F.Cu") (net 2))
 (segment (start 45.62 58) (end 45.5 58) (width 0.25) (layer "F.Cu") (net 2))
 (segment (start 66.62 50.7) (end 66.5 50.75) (width 0.25) (layer "F.Cu") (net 2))
 (segment (start 36.75 41.75) (end 35.25 41.75) (width 0.25) (layer "F.Cu") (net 2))
 (segment (start 36.75 40.5) (end 36.75 41.75) (width 0.25) (layer "F.Cu") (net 2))
 (segment (start 59 48.16) (end 59 48.25) (width 0.25) (layer "F.Cu") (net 2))
 (segment (start 43 53.239999) (end 43 53.25) (width 0.25) (layer "F.Cu") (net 2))
 (segment (start 65.5 50.75) (end 65.5 51.5) (width 0.25) (layer "F.Cu") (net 2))
 (segment (start 66.62 43.08) (end 66.5 43) (width 0.25) (layer "F.Cu") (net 2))
 (segment (start 40.75 57.25) (end 41 57.25) (width 0.25) (layer "F.Cu") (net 2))
 (segment (start 41.54 34) (end 41.5 34) (width 0.25) (layer "F.Cu") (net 2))
 (segment (start 59 45.62) (end 59 45.5) (width 0.25) (layer "F.Cu") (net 2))
 (segment (start 31.75 36.25) (end 36.25 36.25) (width 0.25) (layer "F.Cu") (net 2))
 (segment (start 65 51.5) (end 65 58) (width 0.25) (layer "F.Cu") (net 2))
 (segment (start 35.25 41.75) (end 35.25 42.5) (width 0.25) (layer "F.Cu") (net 2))
 (segment (start 50.62 43.08) (end 50.5 43) (width 0.25) (layer "F.Cu") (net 2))
 (segment (start 60.5 49) (end 60.5 52.25) (width 0.25) (layer "F.Cu") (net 2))
 (segment (start 60.5 52.25) (end 60.5 49) (width 0.25) (layer "F.Cu") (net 2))
 (segment (start 43 43.08) (end 43 43) (width 0.25) (layer "F.Cu") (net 2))
 (segment (start 57.5 35.5) (end 57.5 34) (width 0.25) (layer "F.Cu") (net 2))
 (segment (start 43 40.54) (end 43 40.5) (width 0.25) (layer "F.Cu") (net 2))
 (segment (start 59 45.5) (end 59 48.25) (width 0.25) (layer "F.Cu") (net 2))
 (segment (start 59 48.25) (end 66.5 48.25) (width 0.25) (layer "F.Cu") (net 2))
 (segment (start 59 45.62) (end 59 45.5) (width 0.25) (layer "F.Cu") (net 2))
 (segment (start 43 40.5) (end 36.75 40.5) (width 0.25) (layer "F.Cu") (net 2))
 (segment (start 66.62 48.16) (end 66.5 48.25) (width 0.25) (layer "F.Cu") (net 2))
 (segment (start 59 48.16) (end 59 48.25) (width 0.25) (layer "F.Cu") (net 2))
 (segment (start 66.62 48.16) (end 66.5 48.25) (width 0.25) (layer "F.Cu") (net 2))
 (segment (start 45.62 58) (end 45.5 58) (width 0.25) (layer "F.Cu") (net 2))
 (segment (start 50.5 43) (end 50.5 45.5) (width 0.25) (layer "F.Cu") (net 2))
 (segment (start 40.75 52.25) (end 40.75 57.25) (width 0.25) (layer "F.Cu") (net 2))
 (segment (start 65.62 58) (end 65.5 58) (width 0.25) (layer "F.Cu") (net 2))
 (segment (start 43 53.239999) (end 43 53.25) (width 0.25) (layer "F.Cu") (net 2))
 (via (at 60.25 56.25) (size 0.65) (drill 0.3) (layers "F.Cu" "B.Cu") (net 2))
 (via (at 40 53.25) (size 0.65) (drill 0.3) (layers "F.Cu" "B.Cu") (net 2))
 (via (at 40 52.25) (size 0.65) (drill 0.3) (layers "F.Cu" "B.Cu") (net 2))
 (via (at 42.5 58) (size 0.65) (drill 0.3) (layers "F.Cu" "B.Cu") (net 2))
 (via (at 31.75 37) (size 0.65) (drill 0.3) (layers "F.Cu" "B.Cu") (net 2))
 (via (at 41 58) (size 0.65) (drill 0.3) (layers "F.Cu" "B.Cu") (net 2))
 (segment (start 35.25 42.5) (end 35.25 41.75) (width 0.25) (layer "B.Cu") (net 2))
 (segment (start 44.5 45.5) (end 44.5 52.25) (width 0.25) (layer "B.Cu") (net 2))
 (segment (start 43 44) (end 44.5 44) (width 0.25) (layer "B.Cu") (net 2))
 (segment (start 33.25 41.75) (end 33.25 37) (width 0.25) (layer "B.Cu") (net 2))
 (segment (start 43 53.25) (end 40 53.25) (width 0.25) (layer "B.Cu") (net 2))
 (segment (start 44.5 52.25) (end 40 52.25) (width 0.25) (layer "B.Cu") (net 2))
 (segment (start 43 43) (end 50.5 43) (width 0.25) (layer "B.Cu") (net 2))
 (segment (start 44.5 52.25) (end 43 52.25) (width 0.25) (layer "B.Cu") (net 2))
 (segment (start 43 52.25) (end 43 53.25) (width 0.25) (layer "B.Cu") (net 2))
 (segment (start 50.5 45.5) (end 44.5 45.5) (width 0.25) (layer "B.Cu") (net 2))
 (segment (start 42.5 58) (end 45.5 58) (width 0.25) (layer "B.Cu") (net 2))
 (segment (start 43 43.25) (end 43 44) (width 0.25) (layer "B.Cu") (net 2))
 (segment (start 33.25 37) (end 31.75 37) (width 0.25) (layer "B.Cu") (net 2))
 (segment (start 41 58) (end 41 56.25) (width 0.25) (layer "B.Cu") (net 2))
 (segment (start 44.5 44) (end 44.5 52.25) (width 0.25) (layer "B.Cu") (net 2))
 (segment (start 35.25 41.75) (end 33.25 41.75) (width 0.25) (layer "B.Cu") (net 2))
 (segment (start 41 56.25) (end 60.25 56.25) (width 0.25) (layer "B.Cu") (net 2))
 (segment (start 38 59.5) (end 38 62) (width 0.25) (layer "F.Cu") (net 11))
 (segment (start 39.5 56.5) (end 39.5 59.5) (width 0.25) (layer "F.Cu") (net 11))
 (segment (start 36.75 46) (end 36.75 56.5) (width 0.25) (layer "F.Cu") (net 11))
 (segment (start 35 45) (end 35 46) (width 0.25) (layer "F.Cu") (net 11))
 (segment (start 39.5 59.5) (end 38 59.5) (width 0.25) (layer "F.Cu") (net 11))
 (segment (start 35 45.08) (end 35 45) (width 0.25) (layer "F.Cu") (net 11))
 (segment (start 35 46) (end 36.75 46) (width 0.25) (layer "F.Cu") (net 11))
 (segment (start 36.75 56.5) (end 39.5 56.5) (width 0.25) (layer "F.Cu") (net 11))
 (segment (start 51.25 62) (end 54 62) (width 0.25) (layer "F.Cu") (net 12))
 (segment (start 45.5 59.5) (end 45.5 62) (width 0.25) (layer "F.Cu") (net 12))
 (segment (start 51.25 58) (end 51.25 62) (width 0.25) (layer "F.Cu") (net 12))
 (segment (start 45.62 62) (end 45.5 62) (width 0.25) (layer "F.Cu") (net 12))
 (segment (start 51.25 59.5) (end 45.5 59.5) (width 0.25) (layer "F.Cu") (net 12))
 (segment (start 51.269999 58) (end 51.25 58) (width 0.25) (layer "F.Cu") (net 12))
 (segment (start 51.25 58) (end 51.25 59.5) (width 0.25) (layer "F.Cu") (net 12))
 (segment (start 51.269999 58) (end 51.25 58) (width 0.25) (layer "F.Cu") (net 12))
 (segment (start 44 68) (end 45.5 68) (width 0.25) (layer "F.Cu") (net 6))
 (segment (start 52.5 56.5) (end 44 56.5) (width 0.25) (layer "F.Cu") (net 6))
 (segment (start 43 45.5) (end 43 46.5) (width 0.25) (layer "F.Cu") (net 6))
 (segment (start 43 45.62) (end 43 45.5) (width 0.25) (layer "F.Cu") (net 6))
 (segment (start 52.5 56.5) (end 52.5 58) (width 0.25) (layer "F.Cu") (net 6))
 (segment (start 52.54 58) (end 52.5 58) (width 0.25) (layer "F.Cu") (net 6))
 (segment (start 41.5 46.5) (end 41.5 56.5) (width 0.25) (layer "F.Cu") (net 6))
 (segment (start 43 46.5) (end 41.5 46.5) (width 0.25) (layer "F.Cu") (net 6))
 (segment (start 41.5 56.5) (end 52.5 56.5) (width 0.25) (layer "F.Cu") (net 6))
 (segment (start 44 56.5) (end 44 68) (width 0.25) (layer "F.Cu") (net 6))
 (segment (start 52.5 58) (end 52.5 56.5) (width 0.25) (layer "F.Cu") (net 6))
 (segment (start 45.62 68) (end 45.5 68) (width 0.25) (layer "F.Cu") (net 6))
 (segment (start 52.54 58) (end 52.5 58) (width 0.25) (layer "F.Cu") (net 6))
 (segment (start 61.62 68) (end 61.5 68) (width 0.25) (layer "F.Cu") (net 4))
 (segment (start 33.25 66.5) (end 39.5 66.5) (width 0.25) (layer "F.Cu") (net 4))
 (segment (start 35 50.25) (end 35 49.25) (width 0.25) (layer "F.Cu") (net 4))
 (segment (start 35 49.25) (end 33.25 49.25) (width 0.25) (layer "F.Cu") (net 4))
 (segment (start 35 50.16) (end 35 50.25) (width 0.25) (layer "F.Cu") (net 4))
 (segment (start 35 50.25) (end 35 51) (width 0.25) (layer "F.Cu") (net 4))
 (segment (start 55.5 68) (end 61.5 68) (width 0.25) (layer "F.Cu") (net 4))
 (segment (start 39.5 68) (end 43.25 68) (width 0.25) (layer "F.Cu") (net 4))
 (segment (start 43.25 68.75) (end 44 68.75) (width 0.25) (layer "F.Cu") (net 4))
 (segment (start 35 51) (end 33.25 51) (width 0.25) (layer "F.Cu") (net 4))
 (segment (start 39.5 66.5) (end 39.5 68) (width 0.25) (layer "F.Cu") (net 4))
 (segment (start 35 50.16) (end 35 50.25) (width 0.25) (layer "F.Cu") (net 4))
 (segment (start 33.25 51) (end 33.25 66.5) (width 0.25) (layer "F.Cu") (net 4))
 (segment (start 33.25 38) (end 43 38) (width 0.25) (layer "F.Cu") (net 4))
 (segment (start 44 68.75) (end 44 69.5) (width 0.25) (layer "F.Cu") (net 4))
 (segment (start 55.5 69.5) (end 55.5 68) (width 0.25) (layer "F.Cu") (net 4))
 (segment (start 43.25 68) (end 43.25 68.75) (width 0.25) (layer "F.Cu") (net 4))
 (segment (start 33.25 49.25) (end 33.25 38) (width 0.25) (layer "F.Cu") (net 4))
 (segment (start 44 69.5) (end 55.5 69.5) (width 0.25) (layer "F.Cu") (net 4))
 (segment (start 35 52.75) (end 35 52.5) (width 0.25) (layer "F.Cu") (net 13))
 (segment (start 43 48.16) (end 43 48.25) (width 0.25) (layer "F.Cu") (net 13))
 (segment (start 35 52.7) (end 35 52.75) (width 0.25) (layer "F.Cu") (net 13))
 (segment (start 36.75 48.25) (end 43 48.25) (width 0.25) (layer "B.Cu") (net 13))
 (segment (start 36.75 51.75) (end 36.75 48.25) (width 0.25) (layer "B.Cu") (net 13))
 (segment (start 35 51.75) (end 36.75 51.75) (width 0.25) (layer "B.Cu") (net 13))
 (segment (start 35 52.5) (end 35 51.75) (width 0.25) (layer "B.Cu") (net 13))
 (segment (start 43 50.7) (end 43 50.75) (width 0.25) (layer "F.Cu") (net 7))
 (segment (start 49 36.5) (end 52.25 36.5) (width 0.25) (layer "F.Cu") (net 7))
 (segment (start 49 38) (end 49 36.5) (width 0.25) (layer "F.Cu") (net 7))
 (segment (start 43 49.75) (end 44.5 49.75) (width 0.25) (layer "F.Cu") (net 7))
 (segment (start 44.5 49.75) (end 44.5 38) (width 0.25) (layer "F.Cu") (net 7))
 (segment (start 52.25 36.5) (end 52.25 38) (width 0.25) (layer "F.Cu") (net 7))
 (segment (start 43 50.75) (end 43 49.75) (width 0.25) (layer "F.Cu") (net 7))
 (segment (start 52.25 38) (end 59 38) (width 0.25) (layer "F.Cu") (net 7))
 (segment (start 44.5 38) (end 49 38) (width 0.25) (layer "F.Cu") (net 7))
 (segment (start 59 40.5) (end 58 40.5) (width 0.25) (layer "F.Cu") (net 1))
 (segment (start 58 41.5) (end 57.5 41.5) (width 0.25) (layer "F.Cu") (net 1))
 (segment (start 59 40.54) (end 59 40.5) (width 0.25) (layer "F.Cu") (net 1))
 (segment (start 35 47.62) (end 35 47.5) (width 0.25) (layer "F.Cu") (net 1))
 (segment (start 58 40.5) (end 58 41.5) (width 0.25) (layer "F.Cu") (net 1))
 (segment (start 59 40.54) (end 59 40.5) (width 0.25) (layer "F.Cu") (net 1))
 (segment (start 57.5 41.5) (end 57.5 58) (width 0.25) (layer "F.Cu") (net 1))
 (segment (start 57.5 58) (end 58 58) (width 0.25) (layer "F.Cu") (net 1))
 (segment (start 41.5 36.5) (end 52.25 36.5) (width 0.25) (layer "B.Cu") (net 1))
 (segment (start 36.75 40.5) (end 41.5 40.5) (width 0.25) (layer "B.Cu") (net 1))
 (segment (start 36.75 46.75) (end 36.75 40.5) (width 0.25) (layer "B.Cu") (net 1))
 (segment (start 41.5 40.5) (end 41.5 36.5) (width 0.25) (layer "B.Cu") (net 1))
 (segment (start 52.25 36.5) (end 52.25 40.5) (width 0.25) (layer "B.Cu") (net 1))
 (segment (start 52.25 40.5) (end 59 40.5) (width 0.25) (layer "B.Cu") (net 1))
 (segment (start 35 47.5) (end 35 46.75) (width 0.25) (layer "B.Cu") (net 1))
 (segment (start 35 46.75) (end 36.75 46.75) (width 0.25) (layer "B.Cu") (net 1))
 (segment (start 59 43.08) (end 59 43) (width 0.25) (layer "F.Cu") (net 5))
 (segment (start 35 55.239999) (end 35 55.25) (width 0.25) (layer "F.Cu") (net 5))
 (segment (start 35 55.25) (end 35 58) (width 0.25) (layer "F.Cu") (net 5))
 (segment (start 35 58) (end 38 58) (width 0.25) (layer "F.Cu") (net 5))
 (segment (start 38 54.75) (end 52.25 54.75) (width 0.25) (layer "B.Cu") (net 5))
 (segment (start 52.25 43) (end 59 43) (width 0.25) (layer "B.Cu") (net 5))
 (segment (start 52.25 54.75) (end 52.25 43) (width 0.25) (layer "B.Cu") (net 5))
 (segment (start 38 58) (end 38 54.75) (width 0.25) (layer "B.Cu") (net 5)))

